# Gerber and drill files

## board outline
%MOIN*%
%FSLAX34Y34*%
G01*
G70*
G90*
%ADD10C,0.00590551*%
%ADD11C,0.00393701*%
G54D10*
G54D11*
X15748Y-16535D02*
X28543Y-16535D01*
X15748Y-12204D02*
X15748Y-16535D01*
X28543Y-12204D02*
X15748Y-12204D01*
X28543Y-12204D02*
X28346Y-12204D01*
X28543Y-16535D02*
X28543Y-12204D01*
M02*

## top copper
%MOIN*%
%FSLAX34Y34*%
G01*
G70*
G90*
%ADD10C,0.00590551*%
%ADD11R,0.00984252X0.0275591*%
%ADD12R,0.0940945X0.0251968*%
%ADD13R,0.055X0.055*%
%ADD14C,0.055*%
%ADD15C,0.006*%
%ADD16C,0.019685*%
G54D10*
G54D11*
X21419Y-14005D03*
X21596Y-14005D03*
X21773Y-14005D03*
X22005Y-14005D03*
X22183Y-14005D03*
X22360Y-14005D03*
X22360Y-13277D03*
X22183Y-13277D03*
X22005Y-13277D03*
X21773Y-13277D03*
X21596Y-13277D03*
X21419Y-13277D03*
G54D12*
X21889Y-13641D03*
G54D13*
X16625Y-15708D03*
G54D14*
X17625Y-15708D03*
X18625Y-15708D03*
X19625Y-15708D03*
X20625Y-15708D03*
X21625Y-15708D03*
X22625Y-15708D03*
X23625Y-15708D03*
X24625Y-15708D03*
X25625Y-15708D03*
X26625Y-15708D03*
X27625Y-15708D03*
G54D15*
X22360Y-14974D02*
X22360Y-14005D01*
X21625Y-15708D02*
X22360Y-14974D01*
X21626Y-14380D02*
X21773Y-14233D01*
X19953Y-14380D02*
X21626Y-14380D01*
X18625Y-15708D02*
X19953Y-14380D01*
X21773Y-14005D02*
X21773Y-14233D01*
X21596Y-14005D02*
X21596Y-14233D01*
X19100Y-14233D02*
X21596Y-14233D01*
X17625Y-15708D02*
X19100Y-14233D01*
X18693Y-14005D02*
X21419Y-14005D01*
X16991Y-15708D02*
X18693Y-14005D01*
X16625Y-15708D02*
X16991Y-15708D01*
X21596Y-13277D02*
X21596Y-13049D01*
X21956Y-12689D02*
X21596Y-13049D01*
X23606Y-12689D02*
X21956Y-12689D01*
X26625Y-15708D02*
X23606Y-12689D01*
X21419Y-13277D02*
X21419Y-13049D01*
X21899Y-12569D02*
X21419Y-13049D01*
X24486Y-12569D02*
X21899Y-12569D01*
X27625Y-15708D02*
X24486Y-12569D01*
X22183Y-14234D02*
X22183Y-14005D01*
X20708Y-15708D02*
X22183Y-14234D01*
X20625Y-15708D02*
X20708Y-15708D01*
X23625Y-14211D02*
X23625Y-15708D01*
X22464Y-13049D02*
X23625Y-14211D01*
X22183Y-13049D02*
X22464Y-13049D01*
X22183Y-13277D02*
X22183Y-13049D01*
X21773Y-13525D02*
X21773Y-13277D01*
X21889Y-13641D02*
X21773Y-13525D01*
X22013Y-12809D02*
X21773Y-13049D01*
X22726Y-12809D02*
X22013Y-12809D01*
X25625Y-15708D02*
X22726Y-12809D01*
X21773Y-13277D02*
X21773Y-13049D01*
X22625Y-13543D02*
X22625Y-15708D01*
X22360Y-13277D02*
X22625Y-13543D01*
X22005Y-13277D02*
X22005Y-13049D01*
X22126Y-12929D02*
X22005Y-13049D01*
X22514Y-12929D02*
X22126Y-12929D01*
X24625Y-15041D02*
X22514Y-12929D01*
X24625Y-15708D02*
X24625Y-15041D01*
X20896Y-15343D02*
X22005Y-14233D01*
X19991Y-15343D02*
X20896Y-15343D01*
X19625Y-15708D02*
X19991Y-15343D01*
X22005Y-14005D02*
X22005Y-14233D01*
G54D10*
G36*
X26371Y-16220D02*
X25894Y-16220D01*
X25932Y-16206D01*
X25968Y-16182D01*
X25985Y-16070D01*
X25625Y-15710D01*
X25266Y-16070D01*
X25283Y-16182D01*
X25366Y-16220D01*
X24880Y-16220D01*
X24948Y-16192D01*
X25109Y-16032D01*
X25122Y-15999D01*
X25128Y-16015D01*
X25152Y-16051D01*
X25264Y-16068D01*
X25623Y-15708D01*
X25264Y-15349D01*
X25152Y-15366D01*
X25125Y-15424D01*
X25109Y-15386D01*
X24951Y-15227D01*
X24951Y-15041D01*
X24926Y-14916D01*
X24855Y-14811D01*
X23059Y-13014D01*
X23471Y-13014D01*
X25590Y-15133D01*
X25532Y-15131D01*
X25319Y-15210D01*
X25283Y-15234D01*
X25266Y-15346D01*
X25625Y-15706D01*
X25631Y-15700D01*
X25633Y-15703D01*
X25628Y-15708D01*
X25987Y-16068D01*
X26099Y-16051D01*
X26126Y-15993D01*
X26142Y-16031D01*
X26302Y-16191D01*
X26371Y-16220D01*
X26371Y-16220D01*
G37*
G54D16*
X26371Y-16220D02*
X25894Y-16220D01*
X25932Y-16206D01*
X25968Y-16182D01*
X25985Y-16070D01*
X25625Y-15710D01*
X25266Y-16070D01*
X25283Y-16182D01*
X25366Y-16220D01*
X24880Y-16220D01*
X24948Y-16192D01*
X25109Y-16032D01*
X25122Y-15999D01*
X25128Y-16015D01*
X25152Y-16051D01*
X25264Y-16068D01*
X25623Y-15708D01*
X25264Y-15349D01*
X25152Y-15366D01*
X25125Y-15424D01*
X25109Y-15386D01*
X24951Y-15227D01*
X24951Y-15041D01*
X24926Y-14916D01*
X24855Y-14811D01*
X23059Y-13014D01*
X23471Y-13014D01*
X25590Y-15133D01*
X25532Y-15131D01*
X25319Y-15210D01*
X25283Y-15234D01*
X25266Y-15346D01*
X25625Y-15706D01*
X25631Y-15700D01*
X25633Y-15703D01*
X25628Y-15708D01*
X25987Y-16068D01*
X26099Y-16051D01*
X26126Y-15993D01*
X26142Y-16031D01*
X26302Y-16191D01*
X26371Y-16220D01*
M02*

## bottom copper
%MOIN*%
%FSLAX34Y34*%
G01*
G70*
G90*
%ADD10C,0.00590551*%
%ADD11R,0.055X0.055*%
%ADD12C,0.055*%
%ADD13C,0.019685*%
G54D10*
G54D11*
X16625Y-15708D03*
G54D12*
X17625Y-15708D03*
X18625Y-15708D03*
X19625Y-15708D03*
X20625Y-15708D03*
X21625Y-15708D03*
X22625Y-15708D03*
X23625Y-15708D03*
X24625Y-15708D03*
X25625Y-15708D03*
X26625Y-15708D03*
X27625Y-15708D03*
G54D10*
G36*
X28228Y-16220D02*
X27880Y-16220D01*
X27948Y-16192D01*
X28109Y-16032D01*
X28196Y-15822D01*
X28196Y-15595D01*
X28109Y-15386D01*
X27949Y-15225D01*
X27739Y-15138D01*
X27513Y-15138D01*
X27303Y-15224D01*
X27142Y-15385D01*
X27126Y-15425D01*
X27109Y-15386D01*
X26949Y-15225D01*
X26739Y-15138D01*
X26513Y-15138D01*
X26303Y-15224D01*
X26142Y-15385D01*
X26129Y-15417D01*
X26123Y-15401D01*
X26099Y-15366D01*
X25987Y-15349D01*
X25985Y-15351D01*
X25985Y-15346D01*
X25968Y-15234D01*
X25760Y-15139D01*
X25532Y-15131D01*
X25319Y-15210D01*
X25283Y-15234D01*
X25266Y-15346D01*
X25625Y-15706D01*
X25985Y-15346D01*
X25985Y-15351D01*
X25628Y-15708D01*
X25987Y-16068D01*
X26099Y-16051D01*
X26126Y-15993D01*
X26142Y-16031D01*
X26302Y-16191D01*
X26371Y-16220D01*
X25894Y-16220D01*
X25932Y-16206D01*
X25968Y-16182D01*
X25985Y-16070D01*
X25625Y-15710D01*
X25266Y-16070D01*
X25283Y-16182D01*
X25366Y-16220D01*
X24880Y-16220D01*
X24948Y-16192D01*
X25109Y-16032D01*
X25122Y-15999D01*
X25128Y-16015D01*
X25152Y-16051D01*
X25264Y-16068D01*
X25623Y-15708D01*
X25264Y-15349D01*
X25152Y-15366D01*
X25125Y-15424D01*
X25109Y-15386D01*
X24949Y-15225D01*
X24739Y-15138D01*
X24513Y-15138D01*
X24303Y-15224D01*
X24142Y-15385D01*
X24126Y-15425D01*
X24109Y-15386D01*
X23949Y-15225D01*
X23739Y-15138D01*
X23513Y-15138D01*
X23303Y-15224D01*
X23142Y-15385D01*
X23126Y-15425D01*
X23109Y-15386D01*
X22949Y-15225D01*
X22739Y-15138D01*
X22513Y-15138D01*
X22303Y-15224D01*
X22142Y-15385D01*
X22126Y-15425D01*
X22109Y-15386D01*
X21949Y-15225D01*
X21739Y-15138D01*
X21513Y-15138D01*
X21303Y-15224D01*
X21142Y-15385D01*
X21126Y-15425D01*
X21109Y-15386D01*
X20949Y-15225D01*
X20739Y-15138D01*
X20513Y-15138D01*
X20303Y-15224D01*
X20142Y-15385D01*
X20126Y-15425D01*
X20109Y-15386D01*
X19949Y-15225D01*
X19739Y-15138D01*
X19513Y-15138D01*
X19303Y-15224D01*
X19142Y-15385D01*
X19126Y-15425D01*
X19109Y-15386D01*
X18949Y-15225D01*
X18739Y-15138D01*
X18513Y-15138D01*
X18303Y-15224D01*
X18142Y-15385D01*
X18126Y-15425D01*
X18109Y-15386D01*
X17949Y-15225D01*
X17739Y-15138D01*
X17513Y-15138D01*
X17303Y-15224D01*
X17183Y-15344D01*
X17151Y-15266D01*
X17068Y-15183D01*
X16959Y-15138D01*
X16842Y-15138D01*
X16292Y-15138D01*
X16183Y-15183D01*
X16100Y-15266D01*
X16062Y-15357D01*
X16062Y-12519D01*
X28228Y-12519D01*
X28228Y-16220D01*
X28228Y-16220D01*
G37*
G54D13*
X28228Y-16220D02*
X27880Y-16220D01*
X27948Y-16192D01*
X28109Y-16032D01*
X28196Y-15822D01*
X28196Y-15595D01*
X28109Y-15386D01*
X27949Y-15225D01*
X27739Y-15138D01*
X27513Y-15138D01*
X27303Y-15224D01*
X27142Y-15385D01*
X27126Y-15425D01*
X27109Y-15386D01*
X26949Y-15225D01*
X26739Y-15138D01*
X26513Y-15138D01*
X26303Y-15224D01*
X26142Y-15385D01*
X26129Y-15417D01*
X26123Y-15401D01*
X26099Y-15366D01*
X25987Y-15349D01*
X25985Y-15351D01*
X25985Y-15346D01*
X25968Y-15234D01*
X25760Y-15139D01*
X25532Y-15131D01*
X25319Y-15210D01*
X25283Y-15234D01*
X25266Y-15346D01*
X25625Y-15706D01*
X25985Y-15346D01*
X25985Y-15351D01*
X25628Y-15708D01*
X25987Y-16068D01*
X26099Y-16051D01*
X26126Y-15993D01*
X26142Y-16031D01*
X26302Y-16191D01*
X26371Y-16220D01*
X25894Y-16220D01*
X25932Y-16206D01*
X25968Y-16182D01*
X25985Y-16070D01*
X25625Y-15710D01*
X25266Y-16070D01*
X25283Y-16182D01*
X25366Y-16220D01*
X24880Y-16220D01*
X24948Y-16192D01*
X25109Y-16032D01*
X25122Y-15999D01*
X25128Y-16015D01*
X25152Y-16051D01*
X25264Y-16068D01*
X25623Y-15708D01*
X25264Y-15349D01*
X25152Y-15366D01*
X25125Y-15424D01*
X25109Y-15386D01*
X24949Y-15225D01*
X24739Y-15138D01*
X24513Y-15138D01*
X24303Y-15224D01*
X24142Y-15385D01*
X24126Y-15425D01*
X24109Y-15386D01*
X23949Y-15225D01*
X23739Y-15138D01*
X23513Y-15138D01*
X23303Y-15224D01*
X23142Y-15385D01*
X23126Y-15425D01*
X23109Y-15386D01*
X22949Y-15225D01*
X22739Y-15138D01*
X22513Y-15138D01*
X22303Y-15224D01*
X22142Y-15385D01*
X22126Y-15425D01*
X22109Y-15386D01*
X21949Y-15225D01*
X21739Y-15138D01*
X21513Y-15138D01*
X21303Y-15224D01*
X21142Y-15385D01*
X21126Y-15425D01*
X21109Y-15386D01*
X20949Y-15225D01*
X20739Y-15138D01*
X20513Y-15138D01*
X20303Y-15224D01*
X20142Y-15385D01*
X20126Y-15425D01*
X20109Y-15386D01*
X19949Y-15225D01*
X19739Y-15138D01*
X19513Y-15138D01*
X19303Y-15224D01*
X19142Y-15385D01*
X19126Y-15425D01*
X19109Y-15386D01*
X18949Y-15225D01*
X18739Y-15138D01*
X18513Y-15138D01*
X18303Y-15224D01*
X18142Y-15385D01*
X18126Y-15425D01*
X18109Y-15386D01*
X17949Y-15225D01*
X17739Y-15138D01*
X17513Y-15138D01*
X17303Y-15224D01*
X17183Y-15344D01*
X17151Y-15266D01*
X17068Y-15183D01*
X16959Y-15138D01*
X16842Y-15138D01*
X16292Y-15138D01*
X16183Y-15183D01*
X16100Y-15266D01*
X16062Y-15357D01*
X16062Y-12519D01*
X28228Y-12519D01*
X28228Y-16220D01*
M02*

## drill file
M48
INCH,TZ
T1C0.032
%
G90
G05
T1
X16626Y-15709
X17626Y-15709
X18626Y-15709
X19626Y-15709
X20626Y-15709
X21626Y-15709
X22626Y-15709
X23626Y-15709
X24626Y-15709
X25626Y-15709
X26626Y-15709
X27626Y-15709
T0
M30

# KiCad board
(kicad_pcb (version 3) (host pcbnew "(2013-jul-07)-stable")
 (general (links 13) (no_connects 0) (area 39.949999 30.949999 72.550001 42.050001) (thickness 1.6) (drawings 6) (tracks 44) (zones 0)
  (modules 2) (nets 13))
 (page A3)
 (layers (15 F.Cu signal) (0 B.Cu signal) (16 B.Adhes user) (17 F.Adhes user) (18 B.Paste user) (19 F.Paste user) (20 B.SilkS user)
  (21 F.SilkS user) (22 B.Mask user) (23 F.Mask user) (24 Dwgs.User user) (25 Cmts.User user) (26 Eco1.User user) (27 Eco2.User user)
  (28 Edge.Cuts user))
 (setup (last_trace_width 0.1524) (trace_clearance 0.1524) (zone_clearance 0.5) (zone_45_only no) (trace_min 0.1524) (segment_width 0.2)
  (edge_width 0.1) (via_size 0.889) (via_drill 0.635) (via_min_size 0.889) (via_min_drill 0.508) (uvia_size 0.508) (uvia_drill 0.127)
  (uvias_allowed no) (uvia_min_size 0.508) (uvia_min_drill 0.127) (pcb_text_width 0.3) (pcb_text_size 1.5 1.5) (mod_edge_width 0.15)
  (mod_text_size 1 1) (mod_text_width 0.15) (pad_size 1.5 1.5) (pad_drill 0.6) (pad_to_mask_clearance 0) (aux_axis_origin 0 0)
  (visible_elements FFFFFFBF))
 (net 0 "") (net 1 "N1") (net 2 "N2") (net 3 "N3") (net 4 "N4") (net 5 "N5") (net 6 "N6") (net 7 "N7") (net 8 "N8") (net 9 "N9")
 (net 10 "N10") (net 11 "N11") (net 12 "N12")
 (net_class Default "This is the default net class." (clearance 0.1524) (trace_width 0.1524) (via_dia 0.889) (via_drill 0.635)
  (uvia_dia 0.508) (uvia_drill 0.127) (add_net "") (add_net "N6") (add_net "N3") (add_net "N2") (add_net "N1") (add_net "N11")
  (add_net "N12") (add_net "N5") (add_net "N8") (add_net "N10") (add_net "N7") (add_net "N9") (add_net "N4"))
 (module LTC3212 (layer F.Cu) (at 55.6 34.65)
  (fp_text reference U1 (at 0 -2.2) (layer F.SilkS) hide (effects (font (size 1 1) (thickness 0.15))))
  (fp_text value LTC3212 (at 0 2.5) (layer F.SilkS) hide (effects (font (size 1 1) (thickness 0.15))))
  (pad 1 smd rect (at -1.195 0.925) (size 0.25 0.7) (layers F.Cu F.Paste F.Mask) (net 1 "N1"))
  (pad 2 smd rect (at -0.745 0.925) (size 0.25 0.7) (layers F.Cu F.Paste F.Mask) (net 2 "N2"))
  (pad 3 smd rect (at -0.295 0.925) (size 0.25 0.7) (layers F.Cu F.Paste F.Mask) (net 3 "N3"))
  (pad 4 smd rect (at 0.295 0.925) (size 0.25 0.7) (layers F.Cu F.Paste F.Mask) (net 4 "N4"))
  (pad 5 smd rect (at 0.745 0.925) (size 0.25 0.7) (layers F.Cu F.Paste F.Mask) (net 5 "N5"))
  (pad 6 smd rect (at 1.195 0.925) (size 0.25 0.7) (layers F.Cu F.Paste F.Mask) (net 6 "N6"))
  (pad 7 smd rect (at 1.195 -0.925) (size 0.25 0.7) (layers F.Cu F.Paste F.Mask) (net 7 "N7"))
  (pad 8 smd rect (at 0.745 -0.925) (size 0.25 0.7) (layers F.Cu F.Paste F.Mask) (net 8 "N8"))
  (pad 9 smd rect (at 0.295 -0.925) (size 0.25 0.7) (layers F.Cu F.Paste F.Mask) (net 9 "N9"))
  (pad 10 smd rect (at -0.295 -0.925) (size 0.25 0.7) (layers F.Cu F.Paste F.Mask) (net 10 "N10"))
  (pad 11 smd rect (at -0.745 -0.925) (size 0.25 0.7) (layers F.Cu F.Paste F.Mask) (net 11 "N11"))
  (pad 12 smd rect (at -1.195 -0.925) (size 0.25 0.7) (layers F.Cu F.Paste F.Mask) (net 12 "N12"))
  (pad 13 smd rect (at 0 0) (size 2.39 0.64) (layers F.Cu F.Paste F.Mask) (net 10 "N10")))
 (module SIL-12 (layer F.Cu) (at 56.2 39.9)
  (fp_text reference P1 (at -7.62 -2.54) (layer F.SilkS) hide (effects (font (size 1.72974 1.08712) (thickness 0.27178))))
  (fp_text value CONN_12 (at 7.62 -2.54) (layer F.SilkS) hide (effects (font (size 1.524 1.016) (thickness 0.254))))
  (pad 1 thru_hole rect (at -13.97 0) (size 1.397 1.397) (drill 0.8128) (layers *.Cu *.Mask F.SilkS) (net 1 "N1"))
  (pad 2 thru_hole circle (at -11.43 0) (size 1.397 1.397) (drill 0.8128) (layers *.Cu *.Mask F.SilkS) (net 2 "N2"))
  (pad 3 thru_hole circle (at -8.89 0) (size 1.397 1.397) (drill 0.8128) (layers *.Cu *.Mask F.SilkS) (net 3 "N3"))
  (pad 4 thru_hole circle (at -6.35 0) (size 1.397 1.397) (drill 0.8128) (layers *.Cu *.Mask F.SilkS) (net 4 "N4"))
  (pad 5 thru_hole circle (at -3.81 0) (size 1.397 1.397) (drill 0.8128) (layers *.Cu *.Mask F.SilkS) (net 5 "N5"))
  (pad 6 thru_hole circle (at -1.27 0) (size 1.397 1.397) (drill 0.8128) (layers *.Cu *.Mask F.SilkS) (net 6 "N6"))
  (pad 7 thru_hole circle (at 1.27 0) (size 1.397 1.397) (drill 0.8128) (layers *.Cu *.Mask F.SilkS) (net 7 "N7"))
  (pad 8 thru_hole circle (at 3.81 0) (size 1.397 1.397) (drill 0.8128) (layers *.Cu *.Mask F.SilkS) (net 8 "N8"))
  (pad 9 thru_hole circle (at 6.35 0) (size 1.397 1.397) (drill 0.8128) (layers *.Cu *.Mask F.SilkS) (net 9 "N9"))
  (pad 10 thru_hole circle (at 8.89 0) (size 1.397 1.397) (drill 0.8128) (layers *.Cu *.Mask F.SilkS) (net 10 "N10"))
  (pad 11 thru_hole circle (at 11.43 0) (size 1.397 1.397) (drill 0.8128) (layers *.Cu *.Mask F.SilkS) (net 11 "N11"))
  (pad 12 thru_hole circle (at 13.97 0) (size 1.397 1.397) (drill 0.8128) (layers *.Cu *.Mask F.SilkS) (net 12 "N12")))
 (gr_line (start 40 42) (end 72.5 42) (angle 90) (layer Edge.Cuts) (width 0.1))
 (gr_line (start 40 31) (end 40 42) (angle 90) (layer Edge.Cuts) (width 0.1))
 (gr_line (start 72.5 31) (end 40 31) (angle 90) (layer Edge.Cuts) (width 0.1))
 (gr_line (start 72.5 31) (end 72 31) (angle 90) (layer Edge.Cuts) (width 0.1))
 (gr_line (start 72.5 42) (end 72.5 31) (angle 90) (layer Edge.Cuts) (width 0.1))
 (segment (start 56.795 38.035) (end 56.795 35.575) (width 0.1524) (layer F.Cu) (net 6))
 (segment (start 54.93 39.9) (end 56.795 38.035) (width 0.1524) (layer F.Cu) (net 6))
 (segment (start 54.9319 36.527) (end 55.305 36.1539) (width 0.1524) (layer F.Cu) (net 3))
 (segment (start 50.683 36.527) (end 54.9319 36.527) (width 0.1524) (layer F.Cu) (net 3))
 (segment (start 47.31 39.9) (end 50.683 36.527) (width 0.1524) (layer F.Cu) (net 3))
 (segment (start 55.305 35.575) (end 55.305 36.1539) (width 0.1524) (layer F.Cu) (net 3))
 (segment (start 54.855 35.575) (end 54.855 36.1539) (width 0.1524) (layer F.Cu) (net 2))
 (segment (start 48.5161 36.1539) (end 54.855 36.1539) (width 0.1524) (layer F.Cu) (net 2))
 (segment (start 44.77 39.9) (end 48.5161 36.1539) (width 0.1524) (layer F.Cu) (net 2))
 (segment (start 47.4824 35.575) (end 54.405 35.575) (width 0.1524) (layer F.Cu) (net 1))
 (segment (start 43.1574 39.9) (end 47.4824 35.575) (width 0.1524) (layer F.Cu) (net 1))
 (segment (start 42.23 39.9) (end 43.1574 39.9) (width 0.1524) (layer F.Cu) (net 1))
 (segment (start 54.855 33.725) (end 54.855 33.1461) (width 0.1524) (layer F.Cu) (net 11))
 (segment (start 55.7703 32.2308) (end 54.855 33.1461) (width 0.1524) (layer F.Cu) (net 11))
 (segment (start 59.9608 32.2308) (end 55.7703 32.2308) (width 0.1524) (layer F.Cu) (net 11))
 (segment (start 67.63 39.9) (end 59.9608 32.2308) (width 0.1524) (layer F.Cu) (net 11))
 (segment (start 54.405 33.725) (end 54.405 33.1461) (width 0.1524) (layer F.Cu) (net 12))
 (segment (start 55.6254 31.9257) (end 54.405 33.1461) (width 0.1524) (layer F.Cu) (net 12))
 (segment (start 62.1957 31.9257) (end 55.6254 31.9257) (width 0.1524) (layer F.Cu) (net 12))
 (segment (start 70.17 39.9) (end 62.1957 31.9257) (width 0.1524) (layer F.Cu) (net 12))
 (segment (start 56.345 36.155) (end 56.345 35.575) (width 0.1524) (layer F.Cu) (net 5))
 (segment (start 52.6 39.9) (end 56.345 36.155) (width 0.1524) (layer F.Cu) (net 5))
 (segment (start 52.39 39.9) (end 52.6 39.9) (width 0.1524) (layer F.Cu) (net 5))
 (segment (start 60.01 36.0965) (end 60.01 39.9) (width 0.1524) (layer F.Cu) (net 8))
 (segment (start 57.0596 33.1461) (end 60.01 36.0965) (width 0.1524) (layer F.Cu) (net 8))
 (segment (start 56.345 33.1461) (end 57.0596 33.1461) (width 0.1524) (layer F.Cu) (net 8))
 (segment (start 56.345 33.725) (end 56.345 33.1461) (width 0.1524) (layer F.Cu) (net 8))
 (segment (start 55.305 34.355) (end 55.305 33.725) (width 0.1524) (layer F.Cu) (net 10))
 (segment (start 55.6 34.65) (end 55.305 34.355) (width 0.1524) (layer F.Cu) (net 10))
 (segment (start 55.9152 32.5359) (end 55.305 33.1461) (width 0.1524) (layer F.Cu) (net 10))
 (segment (start 57.7259 32.5359) (end 55.9152 32.5359) (width 0.1524) (layer F.Cu) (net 10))
 (segment (start 65.09 39.9) (end 57.7259 32.5359) (width 0.1524) (layer F.Cu) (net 10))
 (segment (start 55.305 33.725) (end 55.305 33.1461) (width 0.1524) (layer F.Cu) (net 10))
 (segment (start 57.47 34.4) (end 57.47 39.9) (width 0.1524) (layer F.Cu) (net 7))
 (segment (start 56.795 33.725) (end 57.47 34.4) (width 0.1524) (layer F.Cu) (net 7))
 (segment (start 55.895 33.725) (end 55.895 33.1461) (width 0.1524) (layer F.Cu) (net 9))
 (segment (start 56.2001 32.841) (end 55.895 33.1461) (width 0.1524) (layer F.Cu) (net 9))
 (segment (start 57.1861 32.841) (end 56.2001 32.841) (width 0.1524) (layer F.Cu) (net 9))
 (segment (start 62.55 38.2049) (end 57.1861 32.841) (width 0.1524) (layer F.Cu) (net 9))
 (segment (start 62.55 39.9) (end 62.55 38.2049) (width 0.1524) (layer F.Cu) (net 9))
 (segment (start 53.0764 38.9725) (end 55.895 36.1539) (width 0.1524) (layer F.Cu) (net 4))
 (segment (start 50.7775 38.9725) (end 53.0764 38.9725) (width 0.1524) (layer F.Cu) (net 4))
 (segment (start 49.85 39.9) (end 50.7775 38.9725) (width 0.1524) (layer F.Cu) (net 4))
 (segment (start 55.895 35.575) (end 55.895 36.1539) (width 0.1524) (layer F.Cu) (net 4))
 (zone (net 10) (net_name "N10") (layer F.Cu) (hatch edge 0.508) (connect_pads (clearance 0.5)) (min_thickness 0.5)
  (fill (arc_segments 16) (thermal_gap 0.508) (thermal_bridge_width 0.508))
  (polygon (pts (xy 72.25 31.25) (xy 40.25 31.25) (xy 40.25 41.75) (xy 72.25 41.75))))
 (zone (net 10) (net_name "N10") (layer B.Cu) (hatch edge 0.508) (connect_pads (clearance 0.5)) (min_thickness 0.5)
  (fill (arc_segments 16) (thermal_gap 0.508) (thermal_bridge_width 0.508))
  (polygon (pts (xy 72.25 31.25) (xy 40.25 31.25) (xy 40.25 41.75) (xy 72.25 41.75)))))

